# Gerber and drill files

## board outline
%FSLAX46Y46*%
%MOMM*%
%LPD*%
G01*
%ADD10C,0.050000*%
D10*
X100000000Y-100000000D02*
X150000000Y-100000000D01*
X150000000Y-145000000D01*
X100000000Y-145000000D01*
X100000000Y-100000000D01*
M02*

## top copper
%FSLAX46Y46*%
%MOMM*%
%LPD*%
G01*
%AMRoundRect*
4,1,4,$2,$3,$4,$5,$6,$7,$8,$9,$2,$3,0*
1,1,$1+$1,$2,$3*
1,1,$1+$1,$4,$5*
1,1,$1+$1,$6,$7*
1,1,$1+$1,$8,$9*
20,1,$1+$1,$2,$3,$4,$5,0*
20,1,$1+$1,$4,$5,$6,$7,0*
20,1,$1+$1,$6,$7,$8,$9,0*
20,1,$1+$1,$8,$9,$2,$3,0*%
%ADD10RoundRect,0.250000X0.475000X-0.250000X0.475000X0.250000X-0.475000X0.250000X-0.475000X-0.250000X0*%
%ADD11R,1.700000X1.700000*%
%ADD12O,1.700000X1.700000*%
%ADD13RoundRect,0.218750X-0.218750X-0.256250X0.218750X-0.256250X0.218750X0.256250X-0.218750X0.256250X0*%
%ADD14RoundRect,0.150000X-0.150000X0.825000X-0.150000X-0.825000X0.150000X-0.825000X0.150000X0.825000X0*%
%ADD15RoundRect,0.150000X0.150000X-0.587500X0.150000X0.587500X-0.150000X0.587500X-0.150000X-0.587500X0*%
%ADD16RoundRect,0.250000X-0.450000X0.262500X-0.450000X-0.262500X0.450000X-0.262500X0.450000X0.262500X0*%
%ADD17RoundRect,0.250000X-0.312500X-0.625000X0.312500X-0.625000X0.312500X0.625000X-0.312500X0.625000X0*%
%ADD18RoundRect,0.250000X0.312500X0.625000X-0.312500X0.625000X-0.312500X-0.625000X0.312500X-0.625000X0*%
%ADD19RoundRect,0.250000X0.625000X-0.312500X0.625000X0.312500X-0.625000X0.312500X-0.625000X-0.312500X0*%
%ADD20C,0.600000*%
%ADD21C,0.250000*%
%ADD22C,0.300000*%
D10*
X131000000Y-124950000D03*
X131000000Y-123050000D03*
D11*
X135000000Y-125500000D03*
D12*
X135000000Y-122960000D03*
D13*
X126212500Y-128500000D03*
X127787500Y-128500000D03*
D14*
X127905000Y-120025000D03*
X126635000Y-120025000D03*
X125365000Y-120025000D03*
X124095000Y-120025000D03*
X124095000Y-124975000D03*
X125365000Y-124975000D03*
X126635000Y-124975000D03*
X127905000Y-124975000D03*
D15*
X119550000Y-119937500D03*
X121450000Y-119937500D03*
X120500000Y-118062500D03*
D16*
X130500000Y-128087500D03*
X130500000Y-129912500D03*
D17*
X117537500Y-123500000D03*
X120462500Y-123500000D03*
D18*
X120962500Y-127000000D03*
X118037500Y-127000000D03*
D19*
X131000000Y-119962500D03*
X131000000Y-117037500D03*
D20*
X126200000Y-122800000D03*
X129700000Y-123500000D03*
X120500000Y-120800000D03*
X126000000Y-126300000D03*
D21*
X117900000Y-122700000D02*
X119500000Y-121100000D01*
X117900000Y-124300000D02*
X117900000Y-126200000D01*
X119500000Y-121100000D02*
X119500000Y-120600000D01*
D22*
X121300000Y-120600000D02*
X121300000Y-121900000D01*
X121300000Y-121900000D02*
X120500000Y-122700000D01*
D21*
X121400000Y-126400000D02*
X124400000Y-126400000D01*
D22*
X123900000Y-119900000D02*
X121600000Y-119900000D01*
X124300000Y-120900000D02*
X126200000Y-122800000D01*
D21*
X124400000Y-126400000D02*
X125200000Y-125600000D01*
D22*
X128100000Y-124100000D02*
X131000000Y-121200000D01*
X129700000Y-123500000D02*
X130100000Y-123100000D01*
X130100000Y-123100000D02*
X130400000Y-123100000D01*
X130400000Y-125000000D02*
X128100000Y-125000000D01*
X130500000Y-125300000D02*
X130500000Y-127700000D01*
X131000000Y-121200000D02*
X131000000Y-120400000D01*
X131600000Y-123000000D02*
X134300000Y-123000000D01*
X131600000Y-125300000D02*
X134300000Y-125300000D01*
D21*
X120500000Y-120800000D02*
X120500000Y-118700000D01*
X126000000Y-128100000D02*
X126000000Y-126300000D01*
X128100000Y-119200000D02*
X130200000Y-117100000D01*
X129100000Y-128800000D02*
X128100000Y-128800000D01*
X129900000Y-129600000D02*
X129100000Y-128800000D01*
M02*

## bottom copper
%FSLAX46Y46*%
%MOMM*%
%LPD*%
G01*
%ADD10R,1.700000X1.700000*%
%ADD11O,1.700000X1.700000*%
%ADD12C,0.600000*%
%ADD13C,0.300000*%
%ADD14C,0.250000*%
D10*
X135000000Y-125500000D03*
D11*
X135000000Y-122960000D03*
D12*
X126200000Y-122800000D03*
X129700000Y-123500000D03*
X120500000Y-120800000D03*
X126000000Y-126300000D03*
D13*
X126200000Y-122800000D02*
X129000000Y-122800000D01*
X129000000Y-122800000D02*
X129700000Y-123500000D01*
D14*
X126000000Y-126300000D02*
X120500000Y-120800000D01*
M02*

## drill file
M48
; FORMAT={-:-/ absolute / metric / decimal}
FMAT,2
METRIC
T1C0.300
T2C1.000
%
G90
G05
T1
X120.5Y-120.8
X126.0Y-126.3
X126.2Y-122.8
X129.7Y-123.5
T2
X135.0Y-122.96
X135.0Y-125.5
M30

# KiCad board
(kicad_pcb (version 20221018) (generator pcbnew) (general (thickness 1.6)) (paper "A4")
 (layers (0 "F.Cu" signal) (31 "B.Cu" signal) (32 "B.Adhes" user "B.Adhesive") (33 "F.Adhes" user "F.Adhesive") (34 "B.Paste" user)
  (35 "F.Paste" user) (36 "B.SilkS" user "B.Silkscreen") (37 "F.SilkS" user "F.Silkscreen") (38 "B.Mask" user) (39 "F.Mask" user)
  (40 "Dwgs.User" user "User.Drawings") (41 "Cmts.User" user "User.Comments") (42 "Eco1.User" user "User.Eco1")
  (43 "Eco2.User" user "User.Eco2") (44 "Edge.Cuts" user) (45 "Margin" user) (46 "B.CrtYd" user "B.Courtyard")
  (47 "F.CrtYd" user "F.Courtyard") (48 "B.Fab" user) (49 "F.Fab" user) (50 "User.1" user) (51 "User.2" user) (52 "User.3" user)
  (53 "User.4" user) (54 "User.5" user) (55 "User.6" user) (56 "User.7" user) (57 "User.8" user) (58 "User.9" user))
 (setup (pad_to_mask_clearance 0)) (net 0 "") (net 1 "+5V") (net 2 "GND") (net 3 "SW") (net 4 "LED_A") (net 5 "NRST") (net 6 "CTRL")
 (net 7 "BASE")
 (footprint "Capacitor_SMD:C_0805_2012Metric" (layer "F.Cu") (at 131 124 90)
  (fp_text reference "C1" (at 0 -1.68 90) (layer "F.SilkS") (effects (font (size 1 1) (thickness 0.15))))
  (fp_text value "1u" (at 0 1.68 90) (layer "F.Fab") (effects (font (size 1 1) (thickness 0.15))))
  (pad "1" smd roundrect (at -0.95 0 90) (size 1 1.45) (layers "F.Cu" "F.Paste" "F.Mask") (roundrect_rratio 0.25) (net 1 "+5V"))
  (pad "2" smd roundrect (at 0.95 0 90) (size 1 1.45) (layers "F.Cu" "F.Paste" "F.Mask") (roundrect_rratio 0.25) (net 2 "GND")))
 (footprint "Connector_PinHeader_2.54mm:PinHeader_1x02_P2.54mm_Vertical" (layer "F.Cu") (at 135 125.5 180)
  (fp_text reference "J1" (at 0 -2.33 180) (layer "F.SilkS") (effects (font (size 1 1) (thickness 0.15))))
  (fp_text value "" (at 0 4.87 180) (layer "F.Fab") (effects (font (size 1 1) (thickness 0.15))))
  (pad "1" thru_hole rect (at 0 0 180) (size 1.7 1.7) (drill 1) (layers "*.Cu" "*.Mask") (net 1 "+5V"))
  (pad "2" thru_hole oval (at 0 2.54 180) (size 1.7 1.7) (drill 1) (layers "*.Cu" "*.Mask") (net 2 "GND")))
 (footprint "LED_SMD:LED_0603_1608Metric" (layer "F.Cu") (at 127 128.5)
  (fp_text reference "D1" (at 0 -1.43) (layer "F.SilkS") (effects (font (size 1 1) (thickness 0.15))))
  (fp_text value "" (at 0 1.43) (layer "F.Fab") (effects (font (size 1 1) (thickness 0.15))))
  (pad "1" smd roundrect (at -0.7875 0) (size 0.875 0.95) (layers "F.Cu" "F.Paste" "F.Mask") (roundrect_rratio 0.25) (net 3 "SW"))
  (pad "2" smd roundrect (at 0.7875 0) (size 0.875 0.95) (layers "F.Cu" "F.Paste" "F.Mask") (roundrect_rratio 0.25) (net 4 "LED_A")))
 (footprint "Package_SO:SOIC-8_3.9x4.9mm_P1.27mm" (layer "F.Cu") (at 126 122.5 -90)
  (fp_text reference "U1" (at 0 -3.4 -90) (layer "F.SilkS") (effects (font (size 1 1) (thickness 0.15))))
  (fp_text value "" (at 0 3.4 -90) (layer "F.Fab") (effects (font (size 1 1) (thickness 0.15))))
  (pad "1" smd roundrect (at -2.475 -1.905 270) (size 1.95 0.6) (layers "F.Cu" "F.Paste" "F.Mask") (roundrect_rratio 0.25) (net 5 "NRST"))
  (pad "2" smd roundrect (at -2.475 -0.635 270) (size 1.95 0.6) (layers "F.Cu" "F.Paste" "F.Mask") (roundrect_rratio 0.25))
  (pad "3" smd roundrect (at -2.475 0.635 270) (size 1.95 0.6) (layers "F.Cu" "F.Paste" "F.Mask") (roundrect_rratio 0.25))
  (pad "4" smd roundrect (at -2.475 1.905 270) (size 1.95 0.6) (layers "F.Cu" "F.Paste" "F.Mask") (roundrect_rratio 0.25) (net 2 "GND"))
  (pad "5" smd roundrect (at 2.475 1.905 270) (size 1.95 0.6) (layers "F.Cu" "F.Paste" "F.Mask") (roundrect_rratio 0.25))
  (pad "6" smd roundrect (at 2.475 0.635 270) (size 1.95 0.6) (layers "F.Cu" "F.Paste" "F.Mask") (roundrect_rratio 0.25) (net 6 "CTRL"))
  (pad "7" smd roundrect (at 2.475 -0.635 270) (size 1.95 0.6) (layers "F.Cu" "F.Paste" "F.Mask") (roundrect_rratio 0.25))
  (pad "8" smd roundrect (at 2.475 -1.905 270) (size 1.95 0.6) (layers "F.Cu" "F.Paste" "F.Mask") (roundrect_rratio 0.25) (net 1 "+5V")))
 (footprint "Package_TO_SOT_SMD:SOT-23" (layer "F.Cu") (at 120.5 119 90)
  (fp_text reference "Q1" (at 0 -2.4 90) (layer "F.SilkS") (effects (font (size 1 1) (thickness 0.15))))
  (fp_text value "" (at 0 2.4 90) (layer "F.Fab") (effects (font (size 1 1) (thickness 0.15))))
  (pad "1" smd roundrect (at -0.9375 -0.95 90) (size 1.475 0.6) (layers "F.Cu" "F.Paste" "F.Mask") (roundrect_rratio 0.25) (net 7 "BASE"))
  (pad "2" smd roundrect (at -0.9375 0.95 90) (size 1.475 0.6) (layers "F.Cu" "F.Paste" "F.Mask") (roundrect_rratio 0.25) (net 2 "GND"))
  (pad "3" smd roundrect (at 0.9375 0 90) (size 1.475 0.6) (layers "F.Cu" "F.Paste" "F.Mask") (roundrect_rratio 0.25) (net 3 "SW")))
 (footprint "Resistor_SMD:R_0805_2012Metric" (layer "F.Cu") (at 130.5 129 -90)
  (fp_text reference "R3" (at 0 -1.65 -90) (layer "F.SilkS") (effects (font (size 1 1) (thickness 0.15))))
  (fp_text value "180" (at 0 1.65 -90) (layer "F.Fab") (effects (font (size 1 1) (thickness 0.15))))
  (pad "1" smd roundrect (at -0.9125 0 270) (size 1.025 1.4) (layers "F.Cu" "F.Paste" "F.Mask") (roundrect_rratio 0.243902) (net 1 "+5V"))
  (pad "2" smd roundrect (at 0.9125 0 270) (size 1.025 1.4) (layers "F.Cu" "F.Paste" "F.Mask") (roundrect_rratio 0.243902) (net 4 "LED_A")))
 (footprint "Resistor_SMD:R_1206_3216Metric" (layer "F.Cu") (at 119 123.5)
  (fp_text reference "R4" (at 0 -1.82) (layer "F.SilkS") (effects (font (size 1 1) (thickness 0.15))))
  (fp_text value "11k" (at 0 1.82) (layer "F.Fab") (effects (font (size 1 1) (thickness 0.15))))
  (pad "1" smd roundrect (at -1.4625 0) (size 1.125 1.75) (layers "F.Cu" "F.Paste" "F.Mask") (roundrect_rratio 0.222222) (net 7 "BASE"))
  (pad "2" smd roundrect (at 1.4625 0) (size 1.125 1.75) (layers "F.Cu" "F.Paste" "F.Mask") (roundrect_rratio 0.222222) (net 2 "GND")))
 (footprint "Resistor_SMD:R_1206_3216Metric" (layer "F.Cu") (at 119.5 127 180)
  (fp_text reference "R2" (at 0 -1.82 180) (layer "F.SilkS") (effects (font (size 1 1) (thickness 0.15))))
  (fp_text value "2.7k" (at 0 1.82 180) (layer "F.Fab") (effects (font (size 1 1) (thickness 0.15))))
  (pad "1" smd roundrect (at -1.4625 0 180) (size 1.125 1.75) (layers "F.Cu" "F.Paste" "F.Mask") (roundrect_rratio 0.222222) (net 6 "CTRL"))
  (pad "2" smd roundrect (at 1.4625 0 180) (size 1.125 1.75) (layers "F.Cu" "F.Paste" "F.Mask") (roundrect_rratio 0.222222) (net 7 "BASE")))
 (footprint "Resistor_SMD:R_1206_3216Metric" (layer "F.Cu") (at 131 118.5 90)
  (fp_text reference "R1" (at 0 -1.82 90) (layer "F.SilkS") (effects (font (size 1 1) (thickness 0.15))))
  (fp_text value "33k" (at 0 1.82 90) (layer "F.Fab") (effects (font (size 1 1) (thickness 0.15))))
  (pad "1" smd roundrect (at -1.4625 0 90) (size 1.125 1.75) (layers "F.Cu" "F.Paste" "F.Mask") (roundrect_rratio 0.222222) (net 1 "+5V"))
  (pad "2" smd roundrect (at 1.4625 0 90) (size 1.125 1.75) (layers "F.Cu" "F.Paste" "F.Mask") (roundrect_rratio 0.222222) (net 5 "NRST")))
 (gr_rect (start 100 100) (end 150 145) (stroke (width 0.05) (type default)) (fill none) (layer "Edge.Cuts"))
 (segment (start 117.9 122.7) (end 119.5 121.1) (width 0.25) (layer "F.Cu") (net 7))
 (segment (start 117.9 124.3) (end 117.9 126.2) (width 0.25) (layer "F.Cu") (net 7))
 (segment (start 119.5 121.1) (end 119.5 120.6) (width 0.25) (layer "F.Cu") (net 7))
 (segment (start 121.3 120.6) (end 121.3 121.9) (width 0.3) (layer "F.Cu") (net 2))
 (segment (start 121.3 121.9) (end 120.5 122.7) (width 0.3) (layer "F.Cu") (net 2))
 (segment (start 121.4 126.4) (end 124.4 126.4) (width 0.25) (layer "F.Cu") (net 6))
 (segment (start 123.9 119.9) (end 121.6 119.9) (width 0.3) (layer "F.Cu") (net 2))
 (segment (start 124.3 120.9) (end 126.2 122.8) (width 0.3) (layer "F.Cu") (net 2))
 (segment (start 124.4 126.4) (end 125.2 125.6) (width 0.25) (layer "F.Cu") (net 6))
 (segment (start 128.1 124.1) (end 131 121.2) (width 0.3) (layer "F.Cu") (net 1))
 (segment (start 129.7 123.5) (end 130.1 123.1) (width 0.3) (layer "F.Cu") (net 2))
 (segment (start 130.1 123.1) (end 130.4 123.1) (width 0.3) (layer "F.Cu") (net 2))
 (segment (start 130.4 125) (end 128.1 125) (width 0.3) (layer "F.Cu") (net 1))
 (segment (start 130.5 125.3) (end 130.5 127.7) (width 0.3) (layer "F.Cu") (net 1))
 (segment (start 131 121.2) (end 131 120.4) (width 0.3) (layer "F.Cu") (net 1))
 (segment (start 131.6 123) (end 134.3 123) (width 0.3) (layer "F.Cu") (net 2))
 (segment (start 131.6 125.3) (end 134.3 125.3) (width 0.3) (layer "F.Cu") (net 1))
 (via (at 126.2 122.8) (size 0.6) (drill 0.3) (layers "F.Cu" "B.Cu") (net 2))
 (via (at 129.7 123.5) (size 0.6) (drill 0.3) (layers "F.Cu" "B.Cu") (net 2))
 (segment (start 120.5 120.8) (end 120.5 118.7) (width 0.25) (layer "F.Cu") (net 3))
 (segment (start 126 128.1) (end 126 126.3) (width 0.25) (layer "F.Cu") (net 3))
 (segment (start 126.2 122.8) (end 129 122.8) (width 0.3) (layer "B.Cu") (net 2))
 (segment (start 128.1 119.2) (end 130.2 117.1) (width 0.25) (layer "F.Cu") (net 5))
 (segment (start 129 122.8) (end 129.7 123.5) (width 0.3) (layer "B.Cu") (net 2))
 (segment (start 129.1 128.8) (end 128.1 128.8) (width 0.25) (layer "F.Cu") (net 4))
 (segment (start 129.9 129.6) (end 129.1 128.8) (width 0.25) (layer "F.Cu") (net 4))
 (via (at 120.5 120.8) (size 0.6) (drill 0.3) (layers "F.Cu" "B.Cu") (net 3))
 (via (at 126 126.3) (size 0.6) (drill 0.3) (layers "F.Cu" "B.Cu") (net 3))
 (segment (start 126 126.3) (end 120.5 120.8) (width 0.25) (layer "B.Cu") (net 3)))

